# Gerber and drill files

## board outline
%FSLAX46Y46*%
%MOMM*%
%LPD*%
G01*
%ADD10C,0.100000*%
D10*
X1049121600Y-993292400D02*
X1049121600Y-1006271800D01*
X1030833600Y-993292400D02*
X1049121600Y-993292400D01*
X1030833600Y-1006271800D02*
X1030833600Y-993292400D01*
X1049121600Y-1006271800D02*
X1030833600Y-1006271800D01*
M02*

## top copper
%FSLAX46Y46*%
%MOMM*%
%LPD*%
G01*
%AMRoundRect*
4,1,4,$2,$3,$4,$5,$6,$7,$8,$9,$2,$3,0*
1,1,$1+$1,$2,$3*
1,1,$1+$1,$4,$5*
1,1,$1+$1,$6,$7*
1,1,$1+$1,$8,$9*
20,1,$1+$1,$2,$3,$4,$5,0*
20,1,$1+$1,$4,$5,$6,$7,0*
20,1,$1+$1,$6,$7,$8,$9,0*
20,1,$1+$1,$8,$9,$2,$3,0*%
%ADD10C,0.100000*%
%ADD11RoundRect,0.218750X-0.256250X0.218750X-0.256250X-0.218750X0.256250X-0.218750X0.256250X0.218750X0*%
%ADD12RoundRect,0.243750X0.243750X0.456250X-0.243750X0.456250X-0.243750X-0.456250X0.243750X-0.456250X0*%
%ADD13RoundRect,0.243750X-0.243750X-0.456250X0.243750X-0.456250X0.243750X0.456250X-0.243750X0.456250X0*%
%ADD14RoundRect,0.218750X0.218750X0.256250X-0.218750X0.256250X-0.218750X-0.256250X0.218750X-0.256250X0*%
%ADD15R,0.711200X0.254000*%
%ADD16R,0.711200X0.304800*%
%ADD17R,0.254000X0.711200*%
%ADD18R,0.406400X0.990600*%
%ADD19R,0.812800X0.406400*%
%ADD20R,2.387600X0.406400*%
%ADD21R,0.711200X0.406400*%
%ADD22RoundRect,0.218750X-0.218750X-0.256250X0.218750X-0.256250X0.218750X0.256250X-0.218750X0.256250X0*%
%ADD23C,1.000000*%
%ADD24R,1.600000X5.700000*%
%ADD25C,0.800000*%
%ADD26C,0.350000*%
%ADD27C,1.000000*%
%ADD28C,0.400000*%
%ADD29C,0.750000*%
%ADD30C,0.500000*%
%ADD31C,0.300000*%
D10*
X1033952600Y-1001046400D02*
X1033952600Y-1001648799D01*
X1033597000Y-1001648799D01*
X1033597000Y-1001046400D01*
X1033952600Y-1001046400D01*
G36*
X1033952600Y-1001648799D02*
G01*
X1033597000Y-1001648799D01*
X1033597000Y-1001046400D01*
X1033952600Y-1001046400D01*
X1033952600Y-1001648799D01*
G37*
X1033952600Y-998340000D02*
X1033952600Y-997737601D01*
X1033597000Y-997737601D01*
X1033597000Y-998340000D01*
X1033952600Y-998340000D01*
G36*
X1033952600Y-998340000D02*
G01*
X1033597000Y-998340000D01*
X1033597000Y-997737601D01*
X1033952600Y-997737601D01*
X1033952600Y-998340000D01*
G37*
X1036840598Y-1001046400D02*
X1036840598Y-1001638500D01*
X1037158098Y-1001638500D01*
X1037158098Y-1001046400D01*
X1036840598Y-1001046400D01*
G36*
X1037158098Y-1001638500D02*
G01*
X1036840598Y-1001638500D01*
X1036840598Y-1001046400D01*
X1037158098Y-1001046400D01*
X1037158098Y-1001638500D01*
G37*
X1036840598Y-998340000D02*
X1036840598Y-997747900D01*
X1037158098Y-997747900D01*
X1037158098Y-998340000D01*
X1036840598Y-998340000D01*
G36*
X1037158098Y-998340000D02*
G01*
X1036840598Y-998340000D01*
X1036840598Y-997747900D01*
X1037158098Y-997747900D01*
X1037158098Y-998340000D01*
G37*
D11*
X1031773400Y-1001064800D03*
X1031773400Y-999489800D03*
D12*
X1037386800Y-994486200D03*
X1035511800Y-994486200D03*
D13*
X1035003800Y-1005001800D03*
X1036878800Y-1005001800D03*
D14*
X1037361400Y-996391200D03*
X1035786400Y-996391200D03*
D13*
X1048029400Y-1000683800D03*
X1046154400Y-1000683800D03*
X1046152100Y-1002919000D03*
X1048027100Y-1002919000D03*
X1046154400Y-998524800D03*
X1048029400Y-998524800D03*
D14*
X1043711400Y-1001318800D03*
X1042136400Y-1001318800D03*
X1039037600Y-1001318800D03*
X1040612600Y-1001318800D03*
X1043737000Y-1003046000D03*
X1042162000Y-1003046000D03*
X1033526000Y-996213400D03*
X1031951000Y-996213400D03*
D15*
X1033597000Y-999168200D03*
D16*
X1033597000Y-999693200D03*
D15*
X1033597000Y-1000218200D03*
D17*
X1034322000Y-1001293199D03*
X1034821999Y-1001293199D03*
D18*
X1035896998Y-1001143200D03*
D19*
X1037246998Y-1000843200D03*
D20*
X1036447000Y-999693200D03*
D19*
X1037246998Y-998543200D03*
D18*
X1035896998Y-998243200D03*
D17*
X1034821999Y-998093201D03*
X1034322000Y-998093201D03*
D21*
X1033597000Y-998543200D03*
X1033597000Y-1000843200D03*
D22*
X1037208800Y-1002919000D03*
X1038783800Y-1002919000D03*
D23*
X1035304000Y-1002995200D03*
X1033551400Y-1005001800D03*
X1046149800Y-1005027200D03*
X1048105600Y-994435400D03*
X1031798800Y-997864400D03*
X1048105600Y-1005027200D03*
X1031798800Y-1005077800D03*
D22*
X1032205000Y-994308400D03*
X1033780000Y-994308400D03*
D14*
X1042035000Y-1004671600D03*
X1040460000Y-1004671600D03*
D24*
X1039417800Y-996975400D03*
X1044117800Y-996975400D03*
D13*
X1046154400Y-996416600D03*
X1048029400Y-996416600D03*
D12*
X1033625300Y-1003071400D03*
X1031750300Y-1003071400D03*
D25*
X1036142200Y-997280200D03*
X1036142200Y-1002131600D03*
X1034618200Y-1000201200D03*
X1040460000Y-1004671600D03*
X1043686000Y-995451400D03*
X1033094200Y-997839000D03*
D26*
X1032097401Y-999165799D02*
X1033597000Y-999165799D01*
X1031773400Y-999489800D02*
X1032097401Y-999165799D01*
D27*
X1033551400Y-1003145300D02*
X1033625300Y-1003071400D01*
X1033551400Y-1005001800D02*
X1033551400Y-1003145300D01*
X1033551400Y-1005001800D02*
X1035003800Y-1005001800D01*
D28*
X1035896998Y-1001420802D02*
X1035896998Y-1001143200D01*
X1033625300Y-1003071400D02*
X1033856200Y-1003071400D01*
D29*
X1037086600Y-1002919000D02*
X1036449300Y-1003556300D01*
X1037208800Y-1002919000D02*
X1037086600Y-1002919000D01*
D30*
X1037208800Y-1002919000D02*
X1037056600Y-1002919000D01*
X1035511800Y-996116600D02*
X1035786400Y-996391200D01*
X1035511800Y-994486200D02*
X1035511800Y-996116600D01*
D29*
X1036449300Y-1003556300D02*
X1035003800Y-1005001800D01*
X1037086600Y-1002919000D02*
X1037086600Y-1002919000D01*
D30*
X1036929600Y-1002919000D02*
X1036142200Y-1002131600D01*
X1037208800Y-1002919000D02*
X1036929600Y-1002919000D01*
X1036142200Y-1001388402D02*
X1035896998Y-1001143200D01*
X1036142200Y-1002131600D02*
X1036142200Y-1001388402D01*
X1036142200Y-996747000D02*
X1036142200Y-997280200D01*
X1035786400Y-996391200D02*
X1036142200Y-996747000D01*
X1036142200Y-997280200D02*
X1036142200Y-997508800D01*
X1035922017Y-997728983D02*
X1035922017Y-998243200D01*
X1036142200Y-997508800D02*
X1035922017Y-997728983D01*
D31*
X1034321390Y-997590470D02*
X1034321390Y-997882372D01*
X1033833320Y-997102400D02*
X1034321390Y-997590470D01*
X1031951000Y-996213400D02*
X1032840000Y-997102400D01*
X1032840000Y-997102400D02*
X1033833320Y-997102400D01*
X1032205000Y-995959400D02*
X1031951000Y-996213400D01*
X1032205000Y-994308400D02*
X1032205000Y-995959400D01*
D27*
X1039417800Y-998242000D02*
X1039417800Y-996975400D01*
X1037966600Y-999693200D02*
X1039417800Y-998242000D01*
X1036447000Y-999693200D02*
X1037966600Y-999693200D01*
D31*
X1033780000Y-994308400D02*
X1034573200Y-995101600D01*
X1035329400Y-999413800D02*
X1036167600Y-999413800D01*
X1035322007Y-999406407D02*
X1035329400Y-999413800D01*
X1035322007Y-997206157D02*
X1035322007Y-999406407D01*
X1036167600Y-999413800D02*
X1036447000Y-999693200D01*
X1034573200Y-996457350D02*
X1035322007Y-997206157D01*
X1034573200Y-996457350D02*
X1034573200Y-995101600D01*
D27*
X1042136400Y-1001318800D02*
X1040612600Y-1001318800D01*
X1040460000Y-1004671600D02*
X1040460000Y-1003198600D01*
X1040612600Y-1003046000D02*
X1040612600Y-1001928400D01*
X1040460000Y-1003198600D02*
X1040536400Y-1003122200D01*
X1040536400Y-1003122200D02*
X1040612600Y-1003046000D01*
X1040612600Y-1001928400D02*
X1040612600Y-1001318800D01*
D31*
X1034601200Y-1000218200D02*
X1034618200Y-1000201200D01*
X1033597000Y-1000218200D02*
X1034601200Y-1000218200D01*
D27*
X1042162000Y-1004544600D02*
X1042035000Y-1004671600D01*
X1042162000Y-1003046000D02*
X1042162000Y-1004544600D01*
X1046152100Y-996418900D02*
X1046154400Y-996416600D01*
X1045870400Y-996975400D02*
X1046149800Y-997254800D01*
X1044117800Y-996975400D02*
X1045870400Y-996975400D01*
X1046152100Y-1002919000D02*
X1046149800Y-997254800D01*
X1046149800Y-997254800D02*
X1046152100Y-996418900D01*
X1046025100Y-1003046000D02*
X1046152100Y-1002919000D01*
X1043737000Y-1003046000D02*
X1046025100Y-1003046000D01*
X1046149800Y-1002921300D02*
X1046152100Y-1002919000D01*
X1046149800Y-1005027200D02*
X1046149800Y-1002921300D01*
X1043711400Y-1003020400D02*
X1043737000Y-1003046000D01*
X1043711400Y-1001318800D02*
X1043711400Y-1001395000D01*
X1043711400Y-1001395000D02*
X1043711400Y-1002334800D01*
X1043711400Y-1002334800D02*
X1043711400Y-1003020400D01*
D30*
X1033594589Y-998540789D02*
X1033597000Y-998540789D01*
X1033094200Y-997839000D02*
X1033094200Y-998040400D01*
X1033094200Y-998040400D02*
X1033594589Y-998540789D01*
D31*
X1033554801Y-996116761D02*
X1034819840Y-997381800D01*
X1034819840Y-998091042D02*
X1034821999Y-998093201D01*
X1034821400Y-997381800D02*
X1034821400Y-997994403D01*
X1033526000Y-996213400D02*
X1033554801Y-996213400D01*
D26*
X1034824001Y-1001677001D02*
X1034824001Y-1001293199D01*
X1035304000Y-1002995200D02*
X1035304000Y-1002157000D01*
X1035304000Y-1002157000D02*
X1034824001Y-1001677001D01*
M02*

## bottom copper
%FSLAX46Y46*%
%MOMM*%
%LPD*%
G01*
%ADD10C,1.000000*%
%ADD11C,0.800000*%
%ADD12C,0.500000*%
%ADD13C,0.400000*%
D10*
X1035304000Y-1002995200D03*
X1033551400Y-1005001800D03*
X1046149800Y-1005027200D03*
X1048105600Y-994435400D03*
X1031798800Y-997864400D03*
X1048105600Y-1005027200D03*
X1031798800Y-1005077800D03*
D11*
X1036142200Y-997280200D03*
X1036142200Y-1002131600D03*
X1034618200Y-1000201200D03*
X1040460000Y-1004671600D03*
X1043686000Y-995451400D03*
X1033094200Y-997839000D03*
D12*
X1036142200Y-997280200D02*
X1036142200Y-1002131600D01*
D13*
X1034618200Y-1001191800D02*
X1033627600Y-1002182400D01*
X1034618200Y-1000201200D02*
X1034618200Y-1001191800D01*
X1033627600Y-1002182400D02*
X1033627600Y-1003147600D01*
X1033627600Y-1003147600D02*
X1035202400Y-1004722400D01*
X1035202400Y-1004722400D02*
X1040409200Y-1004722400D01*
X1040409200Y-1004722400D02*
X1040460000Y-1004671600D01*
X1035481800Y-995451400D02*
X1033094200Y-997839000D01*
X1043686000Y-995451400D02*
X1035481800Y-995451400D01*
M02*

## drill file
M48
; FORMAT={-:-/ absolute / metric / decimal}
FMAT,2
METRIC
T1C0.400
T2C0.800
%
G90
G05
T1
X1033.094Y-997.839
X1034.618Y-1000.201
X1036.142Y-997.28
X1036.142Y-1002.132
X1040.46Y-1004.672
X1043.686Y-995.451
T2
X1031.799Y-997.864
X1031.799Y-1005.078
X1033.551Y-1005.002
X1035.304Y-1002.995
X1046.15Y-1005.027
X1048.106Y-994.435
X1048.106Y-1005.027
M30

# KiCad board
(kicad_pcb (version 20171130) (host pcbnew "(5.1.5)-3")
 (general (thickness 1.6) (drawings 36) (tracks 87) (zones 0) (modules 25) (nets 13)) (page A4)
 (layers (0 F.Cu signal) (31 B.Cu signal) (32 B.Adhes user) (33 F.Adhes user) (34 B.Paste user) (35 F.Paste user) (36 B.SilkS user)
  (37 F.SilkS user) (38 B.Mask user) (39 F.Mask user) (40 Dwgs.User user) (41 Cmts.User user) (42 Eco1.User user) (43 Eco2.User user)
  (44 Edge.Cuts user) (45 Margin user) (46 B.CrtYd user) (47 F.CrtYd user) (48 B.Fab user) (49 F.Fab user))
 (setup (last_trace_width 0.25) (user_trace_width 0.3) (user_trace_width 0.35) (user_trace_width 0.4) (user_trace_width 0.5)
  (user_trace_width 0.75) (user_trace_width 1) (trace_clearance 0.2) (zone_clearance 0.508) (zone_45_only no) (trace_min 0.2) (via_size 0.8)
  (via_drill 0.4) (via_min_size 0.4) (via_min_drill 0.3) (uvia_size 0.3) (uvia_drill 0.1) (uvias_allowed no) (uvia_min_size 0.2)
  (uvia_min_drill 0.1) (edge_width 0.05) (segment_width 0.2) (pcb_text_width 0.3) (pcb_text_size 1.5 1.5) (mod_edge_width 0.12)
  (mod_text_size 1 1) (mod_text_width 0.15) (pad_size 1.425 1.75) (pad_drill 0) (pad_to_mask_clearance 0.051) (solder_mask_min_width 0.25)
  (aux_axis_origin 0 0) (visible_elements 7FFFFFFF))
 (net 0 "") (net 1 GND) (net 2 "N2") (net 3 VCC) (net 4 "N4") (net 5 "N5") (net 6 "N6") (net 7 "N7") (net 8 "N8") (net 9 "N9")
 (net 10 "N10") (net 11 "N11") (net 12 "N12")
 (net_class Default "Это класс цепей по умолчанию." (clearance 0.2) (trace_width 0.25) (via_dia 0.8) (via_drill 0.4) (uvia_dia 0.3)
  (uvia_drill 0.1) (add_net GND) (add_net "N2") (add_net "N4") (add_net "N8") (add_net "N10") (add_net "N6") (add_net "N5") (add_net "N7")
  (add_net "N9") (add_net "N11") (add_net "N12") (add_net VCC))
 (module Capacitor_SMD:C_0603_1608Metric (layer F.Cu) (at 1031.7734 1000.2773 270)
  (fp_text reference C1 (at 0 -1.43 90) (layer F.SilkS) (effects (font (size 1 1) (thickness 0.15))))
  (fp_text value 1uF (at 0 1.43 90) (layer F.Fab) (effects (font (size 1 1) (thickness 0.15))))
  (pad 2 smd roundrect (at 0.7875 0 270) (size 0.875 0.95) (layers F.Cu F.Paste F.Mask) (roundrect_rratio 0.25) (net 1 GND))
  (pad 1 smd roundrect (at -0.7875 0 270) (size 0.875 0.95) (layers F.Cu F.Paste F.Mask) (roundrect_rratio 0.25) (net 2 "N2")))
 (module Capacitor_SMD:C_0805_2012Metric (layer F.Cu) (at 1036.4493 994.4862 180)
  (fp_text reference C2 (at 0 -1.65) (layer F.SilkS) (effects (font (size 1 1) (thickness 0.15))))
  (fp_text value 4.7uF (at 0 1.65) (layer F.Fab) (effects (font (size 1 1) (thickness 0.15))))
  (pad 1 smd roundrect (at -0.9375 0 180) (size 0.975 1.4) (layers F.Cu F.Paste F.Mask) (roundrect_rratio 0.25) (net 1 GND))
  (pad 2 smd roundrect (at 0.9375 0 180) (size 0.975 1.4) (layers F.Cu F.Paste F.Mask) (roundrect_rratio 0.25) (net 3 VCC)))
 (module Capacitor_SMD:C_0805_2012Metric (layer F.Cu) (at 1035.9413 1005.0018)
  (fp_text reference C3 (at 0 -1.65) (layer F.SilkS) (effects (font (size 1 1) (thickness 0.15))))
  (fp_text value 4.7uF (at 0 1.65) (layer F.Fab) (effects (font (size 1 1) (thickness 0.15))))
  (pad 1 smd roundrect (at -0.9375 0) (size 0.975 1.4) (layers F.Cu F.Paste F.Mask) (roundrect_rratio 0.25) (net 3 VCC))
  (pad 2 smd roundrect (at 0.9375 0) (size 0.975 1.4) (layers F.Cu F.Paste F.Mask) (roundrect_rratio 0.25) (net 1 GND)))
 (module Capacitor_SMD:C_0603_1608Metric (layer F.Cu) (at 1036.5739 996.3912 180)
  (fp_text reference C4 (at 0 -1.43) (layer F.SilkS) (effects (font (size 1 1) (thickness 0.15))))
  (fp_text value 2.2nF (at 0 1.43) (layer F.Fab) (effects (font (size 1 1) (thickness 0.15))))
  (pad 1 smd roundrect (at -0.7875 0 180) (size 0.875 0.95) (layers F.Cu F.Paste F.Mask) (roundrect_rratio 0.25) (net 1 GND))
  (pad 2 smd roundrect (at 0.7875 0 180) (size 0.875 0.95) (layers F.Cu F.Paste F.Mask) (roundrect_rratio 0.25) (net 3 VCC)))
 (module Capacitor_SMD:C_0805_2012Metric (layer F.Cu) (at 1047.0919 1000.6838)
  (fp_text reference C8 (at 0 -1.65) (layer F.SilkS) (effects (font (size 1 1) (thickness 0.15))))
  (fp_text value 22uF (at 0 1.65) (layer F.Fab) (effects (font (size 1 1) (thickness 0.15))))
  (pad 2 smd roundrect (at 0.9375 0) (size 0.975 1.4) (layers F.Cu F.Paste F.Mask) (roundrect_rratio 0.25) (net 1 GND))
  (pad 1 smd roundrect (at -0.9375 0) (size 0.975 1.4) (layers F.Cu F.Paste F.Mask) (roundrect_rratio 0.25) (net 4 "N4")))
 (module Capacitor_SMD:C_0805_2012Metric (layer F.Cu) (at 1047.0896 1002.919)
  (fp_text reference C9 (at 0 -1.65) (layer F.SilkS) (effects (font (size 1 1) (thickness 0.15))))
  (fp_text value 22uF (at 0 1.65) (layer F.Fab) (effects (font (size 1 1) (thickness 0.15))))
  (pad 1 smd roundrect (at -0.9375 0) (size 0.975 1.4) (layers F.Cu F.Paste F.Mask) (roundrect_rratio 0.25) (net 4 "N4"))
  (pad 2 smd roundrect (at 0.9375 0) (size 0.975 1.4) (layers F.Cu F.Paste F.Mask) (roundrect_rratio 0.25) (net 1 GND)))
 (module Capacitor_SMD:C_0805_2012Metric (layer F.Cu) (at 1047.0919 998.5248)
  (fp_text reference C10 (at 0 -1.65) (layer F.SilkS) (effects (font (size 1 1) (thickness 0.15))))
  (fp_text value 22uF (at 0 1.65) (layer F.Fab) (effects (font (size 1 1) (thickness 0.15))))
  (pad 1 smd roundrect (at -0.9375 0) (size 0.975 1.4) (layers F.Cu F.Paste F.Mask) (roundrect_rratio 0.25) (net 4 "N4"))
  (pad 2 smd roundrect (at 0.9375 0) (size 0.975 1.4) (layers F.Cu F.Paste F.Mask) (roundrect_rratio 0.25) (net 1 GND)))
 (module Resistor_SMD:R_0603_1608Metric (layer F.Cu) (at 1042.9239 1001.3188 180)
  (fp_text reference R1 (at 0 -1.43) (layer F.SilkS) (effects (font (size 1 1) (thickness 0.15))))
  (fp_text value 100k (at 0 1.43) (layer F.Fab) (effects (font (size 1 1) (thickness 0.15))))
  (pad 1 smd roundrect (at -0.7875 0 180) (size 0.875 0.95) (layers F.Cu F.Paste F.Mask) (roundrect_rratio 0.25) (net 4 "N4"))
  (pad 2 smd roundrect (at 0.7875 0 180) (size 0.875 0.95) (layers F.Cu F.Paste F.Mask) (roundrect_rratio 0.25) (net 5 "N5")))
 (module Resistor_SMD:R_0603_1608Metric (layer F.Cu) (at 1039.8251 1001.3188 180)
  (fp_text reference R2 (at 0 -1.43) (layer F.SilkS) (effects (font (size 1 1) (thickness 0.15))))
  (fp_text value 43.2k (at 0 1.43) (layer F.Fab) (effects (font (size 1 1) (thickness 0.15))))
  (pad 2 smd roundrect (at 0.7875 0 180) (size 0.875 0.95) (layers F.Cu F.Paste F.Mask) (roundrect_rratio 0.25) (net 1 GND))
  (pad 1 smd roundrect (at -0.7875 0 180) (size 0.875 0.95) (layers F.Cu F.Paste F.Mask) (roundrect_rratio 0.25) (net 5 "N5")))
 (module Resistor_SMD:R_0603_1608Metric (layer F.Cu) (at 1042.9495 1003.046 180)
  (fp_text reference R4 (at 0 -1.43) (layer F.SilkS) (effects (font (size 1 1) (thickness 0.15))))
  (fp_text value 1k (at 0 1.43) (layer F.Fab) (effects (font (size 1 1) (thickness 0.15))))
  (pad 1 smd roundrect (at -0.7875 0 180) (size 0.875 0.95) (layers F.Cu F.Paste F.Mask) (roundrect_rratio 0.25) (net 4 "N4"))
  (pad 2 smd roundrect (at 0.7875 0 180) (size 0.875 0.95) (layers F.Cu F.Paste F.Mask) (roundrect_rratio 0.25) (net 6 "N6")))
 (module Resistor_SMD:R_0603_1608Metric (layer F.Cu) (at 1032.7385 996.2134 180)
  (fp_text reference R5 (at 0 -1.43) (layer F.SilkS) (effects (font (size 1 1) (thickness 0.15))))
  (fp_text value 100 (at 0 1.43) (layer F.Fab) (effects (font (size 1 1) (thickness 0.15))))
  (pad 1 smd roundrect (at -0.7875 0 180) (size 0.875 0.95) (layers F.Cu F.Paste F.Mask) (roundrect_rratio 0.25) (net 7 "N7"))
  (pad 2 smd roundrect (at 0.7875 0 180) (size 0.875 0.95) (layers F.Cu F.Paste F.Mask) (roundrect_rratio 0.25) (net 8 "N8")))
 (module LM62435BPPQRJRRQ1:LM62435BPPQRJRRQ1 (layer F.Cu) (at 1035.446999 999.6932)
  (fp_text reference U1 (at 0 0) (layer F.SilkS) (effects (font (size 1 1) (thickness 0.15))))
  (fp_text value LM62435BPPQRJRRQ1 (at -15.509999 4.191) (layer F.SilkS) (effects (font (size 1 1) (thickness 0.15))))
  (fp_poly (pts (xy -1.494399 1.3532) (xy -1.494399 1.955599) (xy -1.849999 1.955599) (xy -1.849999 1.3532)) (layer F.Cu) (width 0.1))
  (fp_poly (pts (xy -1.494399 -1.3532) (xy -1.494399 -1.955599) (xy -1.849999 -1.955599) (xy -1.849999 -1.3532)) (layer F.Cu) (width 0.1))
  (fp_poly (pts (xy 1.393599 1.3532) (xy 1.393599 1.9453) (xy 1.711099 1.9453) (xy 1.711099 1.3532)) (layer F.Cu) (width 0.1))
  (fp_poly (pts (xy 1.393599 -1.3532) (xy 1.393599 -1.9453) (xy 1.711099 -1.9453) (xy 1.711099 -1.3532)) (layer F.Cu) (width 0.1))
  (pad 2 smd rect (at -1.849999 -0.525 90) (size 0.254 0.7112) (layers F.Cu F.Paste F.Mask) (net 2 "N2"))
  (pad 3 smd rect (at -1.849999 0 90) (size 0.3048 0.7112) (layers F.Cu F.Paste F.Mask) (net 1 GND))
  (pad 4 smd rect (at -1.849999 0.525 90) (size 0.254 0.7112) (layers F.Cu F.Paste F.Mask) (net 5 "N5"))
  (pad 6 smd rect (at -1.124999 1.599999) (size 0.254 0.7112) (layers F.Cu F.Paste F.Mask) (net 1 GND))
  (pad 7 smd rect (at -0.625 1.599999) (size 0.254 0.7112) (layers F.Cu F.Paste F.Mask) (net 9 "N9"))
  (pad 8 smd rect (at 0.449999 1.45) (size 0.4064 0.9906) (layers F.Cu F.Paste F.Mask) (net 3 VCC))
  (pad 9 smd rect (at 1.799999 1.15 90) (size 0.4064 0.8128) (layers F.Cu F.Paste F.Mask) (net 1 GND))
  (pad 10 smd rect (at 1.000001 0 90) (size 0.4064 2.3876) (layers F.Cu F.Paste F.Mask) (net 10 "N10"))
  (pad 11 smd rect (at 1.799999 -1.15 90) (size 0.4064 0.8128) (layers F.Cu F.Paste F.Mask) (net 1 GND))
  (pad 12 smd rect (at 0.449999 -1.45) (size 0.4064 0.9906) (layers F.Cu F.Paste F.Mask) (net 3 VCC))
  (pad 13 smd rect (at -0.625 -1.599999) (size 0.254 0.7112) (layers F.Cu F.Paste F.Mask) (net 7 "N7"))
  (pad 14 smd rect (at -1.124999 -1.599999) (size 0.254 0.7112) (layers F.Cu F.Paste F.Mask) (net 8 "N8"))
  (pad 1 smd rect (at -1.849999 -1.15 90) (size 0.4064 0.7112) (layers F.Cu F.Paste F.Mask) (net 4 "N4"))
  (pad 5 smd rect (at -1.849999 1.15 90) (size 0.4064 0.7112) (layers F.Cu F.Paste F.Mask)))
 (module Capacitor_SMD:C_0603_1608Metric (layer F.Cu) (at 1037.9963 1002.919)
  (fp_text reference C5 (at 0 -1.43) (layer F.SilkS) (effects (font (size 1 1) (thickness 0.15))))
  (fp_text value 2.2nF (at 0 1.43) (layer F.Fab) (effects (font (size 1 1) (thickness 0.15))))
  (pad 1 smd roundrect (at -0.7875 0) (size 0.875 0.95) (layers F.Cu F.Paste F.Mask) (roundrect_rratio 0.25) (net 3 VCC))
  (pad 2 smd roundrect (at 0.7875 0) (size 0.875 0.95) (layers F.Cu F.Paste F.Mask) (roundrect_rratio 0.25) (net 1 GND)))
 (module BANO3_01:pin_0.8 (layer F.Cu) (at 1035.304 1001.3952)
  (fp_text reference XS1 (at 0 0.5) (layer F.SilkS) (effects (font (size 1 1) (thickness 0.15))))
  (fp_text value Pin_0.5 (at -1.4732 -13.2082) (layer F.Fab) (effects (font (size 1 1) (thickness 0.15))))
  (pad 1 thru_hole circle (at 0 1.6) (size 1 1) (drill 0.8) (layers *.Cu *.Mask) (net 9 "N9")))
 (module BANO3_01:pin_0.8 (layer F.Cu) (at 1033.5514 1003.4018)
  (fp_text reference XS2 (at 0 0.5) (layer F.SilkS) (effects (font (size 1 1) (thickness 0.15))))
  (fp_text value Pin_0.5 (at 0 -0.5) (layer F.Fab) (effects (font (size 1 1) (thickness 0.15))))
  (pad 1 thru_hole circle (at 0 1.6) (size 1 1) (drill 0.8) (layers *.Cu *.Mask) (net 3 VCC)))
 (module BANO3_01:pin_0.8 (layer F.Cu) (at 1046.1498 1003.4272)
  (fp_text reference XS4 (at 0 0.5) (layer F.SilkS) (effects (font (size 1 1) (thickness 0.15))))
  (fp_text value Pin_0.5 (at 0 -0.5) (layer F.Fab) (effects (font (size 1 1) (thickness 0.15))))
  (pad 1 thru_hole circle (at 0 1.6) (size 1 1) (drill 0.8) (layers *.Cu *.Mask) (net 4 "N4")))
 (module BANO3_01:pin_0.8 (layer F.Cu) (at 1048.1056 992.8354)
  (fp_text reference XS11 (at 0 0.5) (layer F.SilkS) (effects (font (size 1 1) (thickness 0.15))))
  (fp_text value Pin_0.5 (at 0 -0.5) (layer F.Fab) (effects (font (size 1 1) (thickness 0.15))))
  (pad 1 thru_hole circle (at 0 1.6) (size 1 1) (drill 0.8) (layers *.Cu *.Mask) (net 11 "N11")))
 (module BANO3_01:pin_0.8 (layer F.Cu) (at 1031.7988 996.2644)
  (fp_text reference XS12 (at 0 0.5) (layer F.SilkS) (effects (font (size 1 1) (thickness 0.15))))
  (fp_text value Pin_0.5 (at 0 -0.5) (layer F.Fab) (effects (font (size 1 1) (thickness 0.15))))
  (pad 1 thru_hole circle (at 0 1.6) (size 1 1) (drill 0.8) (layers *.Cu *.Mask) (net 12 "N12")))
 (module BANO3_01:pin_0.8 (layer F.Cu) (at 1048.1056 1003.4272)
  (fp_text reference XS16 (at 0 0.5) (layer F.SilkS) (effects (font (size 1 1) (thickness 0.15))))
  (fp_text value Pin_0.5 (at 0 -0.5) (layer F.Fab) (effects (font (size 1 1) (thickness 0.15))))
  (pad 1 thru_hole circle (at 0 1.6) (size 1 1) (drill 0.8) (layers *.Cu *.Mask) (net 11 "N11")))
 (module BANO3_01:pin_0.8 (layer F.Cu) (at 1031.7988 1003.4778)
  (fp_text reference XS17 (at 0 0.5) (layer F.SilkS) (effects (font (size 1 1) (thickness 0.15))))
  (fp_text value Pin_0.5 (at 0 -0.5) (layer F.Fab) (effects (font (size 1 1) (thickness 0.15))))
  (pad 1 thru_hole circle (at 0 1.6) (size 1 1) (drill 0.8) (layers *.Cu *.Mask) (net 12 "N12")))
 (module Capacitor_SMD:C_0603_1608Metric (layer F.Cu) (at 1032.9925 994.3084)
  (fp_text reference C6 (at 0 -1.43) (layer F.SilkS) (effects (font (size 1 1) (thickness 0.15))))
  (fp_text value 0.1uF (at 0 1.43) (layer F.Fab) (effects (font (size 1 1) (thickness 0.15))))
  (pad 1 smd roundrect (at -0.7875 0) (size 0.875 0.95) (layers F.Cu F.Paste F.Mask) (roundrect_rratio 0.25) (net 8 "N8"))
  (pad 2 smd roundrect (at 0.7875 0) (size 0.875 0.95) (layers F.Cu F.Paste F.Mask) (roundrect_rratio 0.25) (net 10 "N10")))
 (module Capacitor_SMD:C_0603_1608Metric (layer F.Cu) (at 1041.2475 1004.6716 180)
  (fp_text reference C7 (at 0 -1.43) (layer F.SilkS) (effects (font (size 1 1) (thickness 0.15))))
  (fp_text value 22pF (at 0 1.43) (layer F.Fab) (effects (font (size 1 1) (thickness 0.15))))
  (pad 1 smd roundrect (at -0.7875 0 180) (size 0.875 0.95) (layers F.Cu F.Paste F.Mask) (roundrect_rratio 0.25) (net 6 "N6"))
  (pad 2 smd roundrect (at 0.7875 0 180) (size 0.875 0.95) (layers F.Cu F.Paste F.Mask) (roundrect_rratio 0.25) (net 5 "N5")))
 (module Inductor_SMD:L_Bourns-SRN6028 (layer F.Cu) (at 1041.7678 996.9754)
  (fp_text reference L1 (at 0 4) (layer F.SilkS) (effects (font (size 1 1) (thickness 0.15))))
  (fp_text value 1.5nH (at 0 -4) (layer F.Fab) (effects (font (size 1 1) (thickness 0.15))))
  (pad 1 smd rect (at -2.35 0) (size 1.6 5.7) (layers F.Cu F.Paste F.Mask) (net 10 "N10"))
  (pad 2 smd rect (at 2.35 0) (size 1.6 5.7) (layers F.Cu F.Paste F.Mask) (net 4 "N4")))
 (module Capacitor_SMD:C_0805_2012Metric (layer F.Cu) (at 1047.0919 996.4166)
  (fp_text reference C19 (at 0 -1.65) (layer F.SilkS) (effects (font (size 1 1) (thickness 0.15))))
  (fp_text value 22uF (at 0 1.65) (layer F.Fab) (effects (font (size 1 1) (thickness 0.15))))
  (pad 1 smd roundrect (at -0.9375 0) (size 0.975 1.4) (layers F.Cu F.Paste F.Mask) (roundrect_rratio 0.25) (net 4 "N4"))
  (pad 2 smd roundrect (at 0.9375 0) (size 0.975 1.4) (layers F.Cu F.Paste F.Mask) (roundrect_rratio 0.25) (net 1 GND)))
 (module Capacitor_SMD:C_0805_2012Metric (layer F.Cu) (at 1032.6878 1003.0714 180)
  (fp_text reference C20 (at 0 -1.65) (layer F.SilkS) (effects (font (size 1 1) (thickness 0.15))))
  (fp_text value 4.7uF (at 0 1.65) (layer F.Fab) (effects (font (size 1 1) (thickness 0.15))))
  (pad 1 smd roundrect (at -0.9375 0 180) (size 0.975 1.4) (layers F.Cu F.Paste F.Mask) (roundrect_rratio 0.25) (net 3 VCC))
  (pad 2 smd roundrect (at 0.9375 0 180) (size 0.975 1.4) (layers F.Cu F.Paste F.Mask) (roundrect_rratio 0.25) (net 1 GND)))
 (gr_line (start 1049.1216 993.2924) (end 1049.1216 1006.2718) (layer Edge.Cuts) (width 0.1))
 (gr_line (start 1030.8336 993.2924) (end 1049.1216 993.2924) (layer Edge.Cuts) (width 0.1))
 (gr_line (start 1030.8336 1006.2718) (end 1030.8336 993.2924) (layer Edge.Cuts) (width 0.1))
 (gr_line (start 1049.1216 1006.2718) (end 1030.8336 1006.2718) (layer Edge.Cuts) (width 0.1))
 (segment (start 1032.097401 999.165799) (end 1033.597 999.165799) (width 0.35) (layer F.Cu) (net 2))
 (segment (start 1031.7734 999.4898) (end 1032.097401 999.165799) (width 0.35) (layer F.Cu) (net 2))
 (via (at 1036.1422 997.2802) (size 0.8) (drill 0.4) (layers F.Cu B.Cu) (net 3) (status 1000000))
 (segment (start 1033.5514 1003.1453) (end 1033.6253 1003.0714) (width 1) (layer F.Cu) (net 3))
 (segment (start 1033.5514 1005.0018) (end 1033.5514 1003.1453) (width 1) (layer F.Cu) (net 3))
 (segment (start 1033.5514 1005.0018) (end 1035.0038 1005.0018) (width 1) (layer F.Cu) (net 3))
 (segment (start 1035.896998 1001.420802) (end 1035.896998 1001.1432) (width 0.4) (layer F.Cu) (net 3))
 (segment (start 1033.6253 1003.0714) (end 1033.8562 1003.0714) (width 0.4) (layer F.Cu) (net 3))
 (segment (start 1037.0866 1002.919) (end 1036.4493 1003.5563) (width 0.75) (layer F.Cu) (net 3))
 (segment (start 1037.2088 1002.919) (end 1037.0866 1002.919) (width 0.75) (layer F.Cu) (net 3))
 (segment (start 1037.2088 1002.919) (end 1037.0566 1002.919) (width 0.5) (layer F.Cu) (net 3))
 (segment (start 1035.5118 996.1166) (end 1035.7864 996.3912) (width 0.5) (layer F.Cu) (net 3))
 (segment (start 1035.5118 994.4862) (end 1035.5118 996.1166) (width 0.5) (layer F.Cu) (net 3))
 (segment (start 1036.4493 1003.5563) (end 1035.0038 1005.0018) (width 0.75) (layer F.Cu) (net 3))
 (segment (start 1037.0866 1002.919) (end 1037.0866 1002.919) (width 0.75) (layer F.Cu) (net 3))
 (via (at 1036.1422 1002.1316) (size 0.8) (drill 0.4) (layers F.Cu B.Cu) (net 3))
 (segment (start 1036.9296 1002.919) (end 1036.1422 1002.1316) (width 0.5) (layer F.Cu) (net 3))
 (segment (start 1037.2088 1002.919) (end 1036.9296 1002.919) (width 0.5) (layer F.Cu) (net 3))
 (segment (start 1036.1422 1001.388402) (end 1035.896998 1001.1432) (width 0.5) (layer F.Cu) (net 3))
 (segment (start 1036.1422 1002.1316) (end 1036.1422 1001.388402) (width 0.5) (layer F.Cu) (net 3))
 (segment (start 1036.1422 996.747) (end 1036.1422 997.2802) (width 0.5) (layer F.Cu) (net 3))
 (segment (start 1035.7864 996.3912) (end 1036.1422 996.747) (width 0.5) (layer F.Cu) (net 3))
 (segment (start 1036.1422 997.2802) (end 1036.1422 997.5088) (width 0.5) (layer F.Cu) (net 3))
 (segment (start 1035.922017 997.728983) (end 1035.922017 998.2432) (width 0.5) (layer F.Cu) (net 3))
 (segment (start 1036.1422 997.5088) (end 1035.922017 997.728983) (width 0.5) (layer F.Cu) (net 3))
 (segment (start 1036.1422 997.2802) (end 1036.1422 1002.1316) (width 0.5) (layer B.Cu) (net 3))
 (segment (start 1034.32139 997.59047) (end 1034.32139 997.882372) (width 0.3) (layer F.Cu) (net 8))
 (segment (start 1033.83332 997.1024) (end 1034.32139 997.59047) (width 0.3) (layer F.Cu) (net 8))
 (segment (start 1031.951 996.2134) (end 1032.84 997.1024) (width 0.3) (layer F.Cu) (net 8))
 (segment (start 1032.84 997.1024) (end 1033.83332 997.1024) (width 0.3) (layer F.Cu) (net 8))
 (segment (start 1032.205 995.9594) (end 1031.951 996.2134) (width 0.3) (layer F.Cu) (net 8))
 (segment (start 1032.205 994.3084) (end 1032.205 995.9594) (width 0.3) (layer F.Cu) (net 8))
 (segment (start 1039.4178 998.242) (end 1039.4178 996.9754) (width 1) (layer F.Cu) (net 10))
 (segment (start 1037.9666 999.6932) (end 1039.4178 998.242) (width 1) (layer F.Cu) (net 10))
 (segment (start 1036.447 999.6932) (end 1037.9666 999.6932) (width 1) (layer F.Cu) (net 10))
 (segment (start 1033.78 994.3084) (end 1034.5732 995.1016) (width 0.3) (layer F.Cu) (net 10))
 (segment (start 1035.3294 999.4138) (end 1036.1676 999.4138) (width 0.3) (layer F.Cu) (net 10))
 (segment (start 1035.322007 999.406407) (end 1035.3294 999.4138) (width 0.3) (layer F.Cu) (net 10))
 (segment (start 1035.322007 997.206157) (end 1035.322007 999.406407) (width 0.3) (layer F.Cu) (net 10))
 (segment (start 1036.1676 999.4138) (end 1036.447 999.6932) (width 0.3) (layer F.Cu) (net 10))
 (segment (start 1034.5732 996.45735) (end 1035.322007 997.206157) (width 0.3) (layer F.Cu) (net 10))
 (segment (start 1034.5732 996.45735) (end 1034.5732 995.1016) (width 0.3) (layer F.Cu) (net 10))
 (segment (start 1042.1364 1001.3188) (end 1040.6126 1001.3188) (width 1) (layer F.Cu) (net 5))
 (segment (start 1040.46 1004.6716) (end 1040.46 1003.1986) (width 1) (layer F.Cu) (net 5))
 (segment (start 1040.6126 1003.046) (end 1040.6126 1001.9284) (width 1) (layer F.Cu) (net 5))
 (segment (start 1040.46 1003.1986) (end 1040.5364 1003.1222) (width 1) (layer F.Cu) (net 5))
 (segment (start 1040.5364 1003.1222) (end 1040.6126 1003.046) (width 1) (layer F.Cu) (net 5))
 (segment (start 1040.6126 1001.9284) (end 1040.6126 1001.3188) (width 1) (layer F.Cu) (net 5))
 (via (at 1034.6182 1000.2012) (size 0.8) (drill 0.4) (layers F.Cu B.Cu) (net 5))
 (segment (start 1034.6012 1000.2182) (end 1034.6182 1000.2012) (width 0.3) (layer F.Cu) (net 5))
 (segment (start 1033.597 1000.2182) (end 1034.6012 1000.2182) (width 0.3) (layer F.Cu) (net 5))
 (segment (start 1034.6182 1001.1918) (end 1033.6276 1002.1824) (width 0.4) (layer B.Cu) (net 5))
 (segment (start 1034.6182 1000.2012) (end 1034.6182 1001.1918) (width 0.4) (layer B.Cu) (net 5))
 (segment (start 1033.6276 1002.1824) (end 1033.6276 1003.1476) (width 0.4) (layer B.Cu) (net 5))
 (segment (start 1033.6276 1003.1476) (end 1035.2024 1004.7224) (width 0.4) (layer B.Cu) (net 5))
 (via (at 1040.46 1004.6716) (size 0.8) (drill 0.4) (layers F.Cu B.Cu) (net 5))
 (segment (start 1035.2024 1004.7224) (end 1040.4092 1004.7224) (width 0.4) (layer B.Cu) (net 5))
 (segment (start 1040.4092 1004.7224) (end 1040.46 1004.6716) (width 0.4) (layer B.Cu) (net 5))
 (segment (start 1042.162 1004.5446) (end 1042.035 1004.6716) (width 1) (layer F.Cu) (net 6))
 (segment (start 1042.162 1003.046) (end 1042.162 1004.5446) (width 1) (layer F.Cu) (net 6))
 (segment (start 1046.1521 996.4189) (end 1046.1544 996.4166) (width 1) (layer F.Cu) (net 4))
 (segment (start 1045.8704 996.9754) (end 1046.1498 997.2548) (width 1) (layer F.Cu) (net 4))
 (segment (start 1044.1178 996.9754) (end 1045.8704 996.9754) (width 1) (layer F.Cu) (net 4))
 (segment (start 1046.1521 1002.919) (end 1046.1498 997.2548) (width 1) (layer F.Cu) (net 4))
 (segment (start 1046.1498 997.2548) (end 1046.1521 996.4189) (width 1) (layer F.Cu) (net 4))
 (segment (start 1046.0251 1003.046) (end 1046.1521 1002.919) (width 1) (layer F.Cu) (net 4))
 (segment (start 1043.737 1003.046) (end 1046.0251 1003.046) (width 1) (layer F.Cu) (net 4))
 (segment (start 1046.1498 1002.9213) (end 1046.1521 1002.919) (width 1) (layer F.Cu) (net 4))
 (segment (start 1046.1498 1005.0272) (end 1046.1498 1002.9213) (width 1) (layer F.Cu) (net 4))
 (segment (start 1043.7114 1003.0204) (end 1043.737 1003.046) (width 1) (layer F.Cu) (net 4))
 (segment (start 1043.7114 1001.3188) (end 1043.7114 1001.395) (width 1) (layer F.Cu) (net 4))
 (segment (start 1043.7114 1001.395) (end 1043.7114 1002.3348) (width 1) (layer F.Cu) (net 4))
 (via (at 1043.686 995.4514) (size 0.8) (drill 0.4) (layers F.Cu B.Cu) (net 4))
 (segment (start 1043.7114 1002.3348) (end 1043.7114 1003.0204) (width 1) (layer F.Cu) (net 4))
 (via (at 1033.0942 997.839) (size 0.8) (drill 0.4) (layers F.Cu B.Cu) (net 4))
 (segment (start 1033.594589 998.540789) (end 1033.597 998.540789) (width 0.5) (layer F.Cu) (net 4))
 (segment (start 1033.0942 997.839) (end 1033.0942 998.0404) (width 0.5) (layer F.Cu) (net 4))
 (segment (start 1033.0942 998.0404) (end 1033.594589 998.540789) (width 0.5) (layer F.Cu) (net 4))
 (segment (start 1035.4818 995.4514) (end 1033.0942 997.839) (width 0.4) (layer B.Cu) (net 4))
 (segment (start 1043.686 995.4514) (end 1035.4818 995.4514) (width 0.4) (layer B.Cu) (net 4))
 (segment (start 1033.554801 996.116761) (end 1034.81984 997.3818) (width 0.3) (layer F.Cu) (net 7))
 (segment (start 1034.81984 998.091042) (end 1034.821999 998.093201) (width 0.3) (layer F.Cu) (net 7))
 (segment (start 1034.8214 997.3818) (end 1034.8214 997.994403) (width 0.3) (layer F.Cu) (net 7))
 (segment (start 1033.526 996.2134) (end 1033.554801 996.2134) (width 0.3) (layer F.Cu) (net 7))
 (segment (start 1034.824001 1001.677001) (end 1034.824001 1001.293199) (width 0.35) (layer F.Cu) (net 9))
 (segment (start 1035.304 1002.9952) (end 1035.304 1002.157) (width 0.35) (layer F.Cu) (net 9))
 (segment (start 1035.304 1002.157) (end 1034.824001 1001.677001) (width 0.35) (layer F.Cu) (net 9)))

